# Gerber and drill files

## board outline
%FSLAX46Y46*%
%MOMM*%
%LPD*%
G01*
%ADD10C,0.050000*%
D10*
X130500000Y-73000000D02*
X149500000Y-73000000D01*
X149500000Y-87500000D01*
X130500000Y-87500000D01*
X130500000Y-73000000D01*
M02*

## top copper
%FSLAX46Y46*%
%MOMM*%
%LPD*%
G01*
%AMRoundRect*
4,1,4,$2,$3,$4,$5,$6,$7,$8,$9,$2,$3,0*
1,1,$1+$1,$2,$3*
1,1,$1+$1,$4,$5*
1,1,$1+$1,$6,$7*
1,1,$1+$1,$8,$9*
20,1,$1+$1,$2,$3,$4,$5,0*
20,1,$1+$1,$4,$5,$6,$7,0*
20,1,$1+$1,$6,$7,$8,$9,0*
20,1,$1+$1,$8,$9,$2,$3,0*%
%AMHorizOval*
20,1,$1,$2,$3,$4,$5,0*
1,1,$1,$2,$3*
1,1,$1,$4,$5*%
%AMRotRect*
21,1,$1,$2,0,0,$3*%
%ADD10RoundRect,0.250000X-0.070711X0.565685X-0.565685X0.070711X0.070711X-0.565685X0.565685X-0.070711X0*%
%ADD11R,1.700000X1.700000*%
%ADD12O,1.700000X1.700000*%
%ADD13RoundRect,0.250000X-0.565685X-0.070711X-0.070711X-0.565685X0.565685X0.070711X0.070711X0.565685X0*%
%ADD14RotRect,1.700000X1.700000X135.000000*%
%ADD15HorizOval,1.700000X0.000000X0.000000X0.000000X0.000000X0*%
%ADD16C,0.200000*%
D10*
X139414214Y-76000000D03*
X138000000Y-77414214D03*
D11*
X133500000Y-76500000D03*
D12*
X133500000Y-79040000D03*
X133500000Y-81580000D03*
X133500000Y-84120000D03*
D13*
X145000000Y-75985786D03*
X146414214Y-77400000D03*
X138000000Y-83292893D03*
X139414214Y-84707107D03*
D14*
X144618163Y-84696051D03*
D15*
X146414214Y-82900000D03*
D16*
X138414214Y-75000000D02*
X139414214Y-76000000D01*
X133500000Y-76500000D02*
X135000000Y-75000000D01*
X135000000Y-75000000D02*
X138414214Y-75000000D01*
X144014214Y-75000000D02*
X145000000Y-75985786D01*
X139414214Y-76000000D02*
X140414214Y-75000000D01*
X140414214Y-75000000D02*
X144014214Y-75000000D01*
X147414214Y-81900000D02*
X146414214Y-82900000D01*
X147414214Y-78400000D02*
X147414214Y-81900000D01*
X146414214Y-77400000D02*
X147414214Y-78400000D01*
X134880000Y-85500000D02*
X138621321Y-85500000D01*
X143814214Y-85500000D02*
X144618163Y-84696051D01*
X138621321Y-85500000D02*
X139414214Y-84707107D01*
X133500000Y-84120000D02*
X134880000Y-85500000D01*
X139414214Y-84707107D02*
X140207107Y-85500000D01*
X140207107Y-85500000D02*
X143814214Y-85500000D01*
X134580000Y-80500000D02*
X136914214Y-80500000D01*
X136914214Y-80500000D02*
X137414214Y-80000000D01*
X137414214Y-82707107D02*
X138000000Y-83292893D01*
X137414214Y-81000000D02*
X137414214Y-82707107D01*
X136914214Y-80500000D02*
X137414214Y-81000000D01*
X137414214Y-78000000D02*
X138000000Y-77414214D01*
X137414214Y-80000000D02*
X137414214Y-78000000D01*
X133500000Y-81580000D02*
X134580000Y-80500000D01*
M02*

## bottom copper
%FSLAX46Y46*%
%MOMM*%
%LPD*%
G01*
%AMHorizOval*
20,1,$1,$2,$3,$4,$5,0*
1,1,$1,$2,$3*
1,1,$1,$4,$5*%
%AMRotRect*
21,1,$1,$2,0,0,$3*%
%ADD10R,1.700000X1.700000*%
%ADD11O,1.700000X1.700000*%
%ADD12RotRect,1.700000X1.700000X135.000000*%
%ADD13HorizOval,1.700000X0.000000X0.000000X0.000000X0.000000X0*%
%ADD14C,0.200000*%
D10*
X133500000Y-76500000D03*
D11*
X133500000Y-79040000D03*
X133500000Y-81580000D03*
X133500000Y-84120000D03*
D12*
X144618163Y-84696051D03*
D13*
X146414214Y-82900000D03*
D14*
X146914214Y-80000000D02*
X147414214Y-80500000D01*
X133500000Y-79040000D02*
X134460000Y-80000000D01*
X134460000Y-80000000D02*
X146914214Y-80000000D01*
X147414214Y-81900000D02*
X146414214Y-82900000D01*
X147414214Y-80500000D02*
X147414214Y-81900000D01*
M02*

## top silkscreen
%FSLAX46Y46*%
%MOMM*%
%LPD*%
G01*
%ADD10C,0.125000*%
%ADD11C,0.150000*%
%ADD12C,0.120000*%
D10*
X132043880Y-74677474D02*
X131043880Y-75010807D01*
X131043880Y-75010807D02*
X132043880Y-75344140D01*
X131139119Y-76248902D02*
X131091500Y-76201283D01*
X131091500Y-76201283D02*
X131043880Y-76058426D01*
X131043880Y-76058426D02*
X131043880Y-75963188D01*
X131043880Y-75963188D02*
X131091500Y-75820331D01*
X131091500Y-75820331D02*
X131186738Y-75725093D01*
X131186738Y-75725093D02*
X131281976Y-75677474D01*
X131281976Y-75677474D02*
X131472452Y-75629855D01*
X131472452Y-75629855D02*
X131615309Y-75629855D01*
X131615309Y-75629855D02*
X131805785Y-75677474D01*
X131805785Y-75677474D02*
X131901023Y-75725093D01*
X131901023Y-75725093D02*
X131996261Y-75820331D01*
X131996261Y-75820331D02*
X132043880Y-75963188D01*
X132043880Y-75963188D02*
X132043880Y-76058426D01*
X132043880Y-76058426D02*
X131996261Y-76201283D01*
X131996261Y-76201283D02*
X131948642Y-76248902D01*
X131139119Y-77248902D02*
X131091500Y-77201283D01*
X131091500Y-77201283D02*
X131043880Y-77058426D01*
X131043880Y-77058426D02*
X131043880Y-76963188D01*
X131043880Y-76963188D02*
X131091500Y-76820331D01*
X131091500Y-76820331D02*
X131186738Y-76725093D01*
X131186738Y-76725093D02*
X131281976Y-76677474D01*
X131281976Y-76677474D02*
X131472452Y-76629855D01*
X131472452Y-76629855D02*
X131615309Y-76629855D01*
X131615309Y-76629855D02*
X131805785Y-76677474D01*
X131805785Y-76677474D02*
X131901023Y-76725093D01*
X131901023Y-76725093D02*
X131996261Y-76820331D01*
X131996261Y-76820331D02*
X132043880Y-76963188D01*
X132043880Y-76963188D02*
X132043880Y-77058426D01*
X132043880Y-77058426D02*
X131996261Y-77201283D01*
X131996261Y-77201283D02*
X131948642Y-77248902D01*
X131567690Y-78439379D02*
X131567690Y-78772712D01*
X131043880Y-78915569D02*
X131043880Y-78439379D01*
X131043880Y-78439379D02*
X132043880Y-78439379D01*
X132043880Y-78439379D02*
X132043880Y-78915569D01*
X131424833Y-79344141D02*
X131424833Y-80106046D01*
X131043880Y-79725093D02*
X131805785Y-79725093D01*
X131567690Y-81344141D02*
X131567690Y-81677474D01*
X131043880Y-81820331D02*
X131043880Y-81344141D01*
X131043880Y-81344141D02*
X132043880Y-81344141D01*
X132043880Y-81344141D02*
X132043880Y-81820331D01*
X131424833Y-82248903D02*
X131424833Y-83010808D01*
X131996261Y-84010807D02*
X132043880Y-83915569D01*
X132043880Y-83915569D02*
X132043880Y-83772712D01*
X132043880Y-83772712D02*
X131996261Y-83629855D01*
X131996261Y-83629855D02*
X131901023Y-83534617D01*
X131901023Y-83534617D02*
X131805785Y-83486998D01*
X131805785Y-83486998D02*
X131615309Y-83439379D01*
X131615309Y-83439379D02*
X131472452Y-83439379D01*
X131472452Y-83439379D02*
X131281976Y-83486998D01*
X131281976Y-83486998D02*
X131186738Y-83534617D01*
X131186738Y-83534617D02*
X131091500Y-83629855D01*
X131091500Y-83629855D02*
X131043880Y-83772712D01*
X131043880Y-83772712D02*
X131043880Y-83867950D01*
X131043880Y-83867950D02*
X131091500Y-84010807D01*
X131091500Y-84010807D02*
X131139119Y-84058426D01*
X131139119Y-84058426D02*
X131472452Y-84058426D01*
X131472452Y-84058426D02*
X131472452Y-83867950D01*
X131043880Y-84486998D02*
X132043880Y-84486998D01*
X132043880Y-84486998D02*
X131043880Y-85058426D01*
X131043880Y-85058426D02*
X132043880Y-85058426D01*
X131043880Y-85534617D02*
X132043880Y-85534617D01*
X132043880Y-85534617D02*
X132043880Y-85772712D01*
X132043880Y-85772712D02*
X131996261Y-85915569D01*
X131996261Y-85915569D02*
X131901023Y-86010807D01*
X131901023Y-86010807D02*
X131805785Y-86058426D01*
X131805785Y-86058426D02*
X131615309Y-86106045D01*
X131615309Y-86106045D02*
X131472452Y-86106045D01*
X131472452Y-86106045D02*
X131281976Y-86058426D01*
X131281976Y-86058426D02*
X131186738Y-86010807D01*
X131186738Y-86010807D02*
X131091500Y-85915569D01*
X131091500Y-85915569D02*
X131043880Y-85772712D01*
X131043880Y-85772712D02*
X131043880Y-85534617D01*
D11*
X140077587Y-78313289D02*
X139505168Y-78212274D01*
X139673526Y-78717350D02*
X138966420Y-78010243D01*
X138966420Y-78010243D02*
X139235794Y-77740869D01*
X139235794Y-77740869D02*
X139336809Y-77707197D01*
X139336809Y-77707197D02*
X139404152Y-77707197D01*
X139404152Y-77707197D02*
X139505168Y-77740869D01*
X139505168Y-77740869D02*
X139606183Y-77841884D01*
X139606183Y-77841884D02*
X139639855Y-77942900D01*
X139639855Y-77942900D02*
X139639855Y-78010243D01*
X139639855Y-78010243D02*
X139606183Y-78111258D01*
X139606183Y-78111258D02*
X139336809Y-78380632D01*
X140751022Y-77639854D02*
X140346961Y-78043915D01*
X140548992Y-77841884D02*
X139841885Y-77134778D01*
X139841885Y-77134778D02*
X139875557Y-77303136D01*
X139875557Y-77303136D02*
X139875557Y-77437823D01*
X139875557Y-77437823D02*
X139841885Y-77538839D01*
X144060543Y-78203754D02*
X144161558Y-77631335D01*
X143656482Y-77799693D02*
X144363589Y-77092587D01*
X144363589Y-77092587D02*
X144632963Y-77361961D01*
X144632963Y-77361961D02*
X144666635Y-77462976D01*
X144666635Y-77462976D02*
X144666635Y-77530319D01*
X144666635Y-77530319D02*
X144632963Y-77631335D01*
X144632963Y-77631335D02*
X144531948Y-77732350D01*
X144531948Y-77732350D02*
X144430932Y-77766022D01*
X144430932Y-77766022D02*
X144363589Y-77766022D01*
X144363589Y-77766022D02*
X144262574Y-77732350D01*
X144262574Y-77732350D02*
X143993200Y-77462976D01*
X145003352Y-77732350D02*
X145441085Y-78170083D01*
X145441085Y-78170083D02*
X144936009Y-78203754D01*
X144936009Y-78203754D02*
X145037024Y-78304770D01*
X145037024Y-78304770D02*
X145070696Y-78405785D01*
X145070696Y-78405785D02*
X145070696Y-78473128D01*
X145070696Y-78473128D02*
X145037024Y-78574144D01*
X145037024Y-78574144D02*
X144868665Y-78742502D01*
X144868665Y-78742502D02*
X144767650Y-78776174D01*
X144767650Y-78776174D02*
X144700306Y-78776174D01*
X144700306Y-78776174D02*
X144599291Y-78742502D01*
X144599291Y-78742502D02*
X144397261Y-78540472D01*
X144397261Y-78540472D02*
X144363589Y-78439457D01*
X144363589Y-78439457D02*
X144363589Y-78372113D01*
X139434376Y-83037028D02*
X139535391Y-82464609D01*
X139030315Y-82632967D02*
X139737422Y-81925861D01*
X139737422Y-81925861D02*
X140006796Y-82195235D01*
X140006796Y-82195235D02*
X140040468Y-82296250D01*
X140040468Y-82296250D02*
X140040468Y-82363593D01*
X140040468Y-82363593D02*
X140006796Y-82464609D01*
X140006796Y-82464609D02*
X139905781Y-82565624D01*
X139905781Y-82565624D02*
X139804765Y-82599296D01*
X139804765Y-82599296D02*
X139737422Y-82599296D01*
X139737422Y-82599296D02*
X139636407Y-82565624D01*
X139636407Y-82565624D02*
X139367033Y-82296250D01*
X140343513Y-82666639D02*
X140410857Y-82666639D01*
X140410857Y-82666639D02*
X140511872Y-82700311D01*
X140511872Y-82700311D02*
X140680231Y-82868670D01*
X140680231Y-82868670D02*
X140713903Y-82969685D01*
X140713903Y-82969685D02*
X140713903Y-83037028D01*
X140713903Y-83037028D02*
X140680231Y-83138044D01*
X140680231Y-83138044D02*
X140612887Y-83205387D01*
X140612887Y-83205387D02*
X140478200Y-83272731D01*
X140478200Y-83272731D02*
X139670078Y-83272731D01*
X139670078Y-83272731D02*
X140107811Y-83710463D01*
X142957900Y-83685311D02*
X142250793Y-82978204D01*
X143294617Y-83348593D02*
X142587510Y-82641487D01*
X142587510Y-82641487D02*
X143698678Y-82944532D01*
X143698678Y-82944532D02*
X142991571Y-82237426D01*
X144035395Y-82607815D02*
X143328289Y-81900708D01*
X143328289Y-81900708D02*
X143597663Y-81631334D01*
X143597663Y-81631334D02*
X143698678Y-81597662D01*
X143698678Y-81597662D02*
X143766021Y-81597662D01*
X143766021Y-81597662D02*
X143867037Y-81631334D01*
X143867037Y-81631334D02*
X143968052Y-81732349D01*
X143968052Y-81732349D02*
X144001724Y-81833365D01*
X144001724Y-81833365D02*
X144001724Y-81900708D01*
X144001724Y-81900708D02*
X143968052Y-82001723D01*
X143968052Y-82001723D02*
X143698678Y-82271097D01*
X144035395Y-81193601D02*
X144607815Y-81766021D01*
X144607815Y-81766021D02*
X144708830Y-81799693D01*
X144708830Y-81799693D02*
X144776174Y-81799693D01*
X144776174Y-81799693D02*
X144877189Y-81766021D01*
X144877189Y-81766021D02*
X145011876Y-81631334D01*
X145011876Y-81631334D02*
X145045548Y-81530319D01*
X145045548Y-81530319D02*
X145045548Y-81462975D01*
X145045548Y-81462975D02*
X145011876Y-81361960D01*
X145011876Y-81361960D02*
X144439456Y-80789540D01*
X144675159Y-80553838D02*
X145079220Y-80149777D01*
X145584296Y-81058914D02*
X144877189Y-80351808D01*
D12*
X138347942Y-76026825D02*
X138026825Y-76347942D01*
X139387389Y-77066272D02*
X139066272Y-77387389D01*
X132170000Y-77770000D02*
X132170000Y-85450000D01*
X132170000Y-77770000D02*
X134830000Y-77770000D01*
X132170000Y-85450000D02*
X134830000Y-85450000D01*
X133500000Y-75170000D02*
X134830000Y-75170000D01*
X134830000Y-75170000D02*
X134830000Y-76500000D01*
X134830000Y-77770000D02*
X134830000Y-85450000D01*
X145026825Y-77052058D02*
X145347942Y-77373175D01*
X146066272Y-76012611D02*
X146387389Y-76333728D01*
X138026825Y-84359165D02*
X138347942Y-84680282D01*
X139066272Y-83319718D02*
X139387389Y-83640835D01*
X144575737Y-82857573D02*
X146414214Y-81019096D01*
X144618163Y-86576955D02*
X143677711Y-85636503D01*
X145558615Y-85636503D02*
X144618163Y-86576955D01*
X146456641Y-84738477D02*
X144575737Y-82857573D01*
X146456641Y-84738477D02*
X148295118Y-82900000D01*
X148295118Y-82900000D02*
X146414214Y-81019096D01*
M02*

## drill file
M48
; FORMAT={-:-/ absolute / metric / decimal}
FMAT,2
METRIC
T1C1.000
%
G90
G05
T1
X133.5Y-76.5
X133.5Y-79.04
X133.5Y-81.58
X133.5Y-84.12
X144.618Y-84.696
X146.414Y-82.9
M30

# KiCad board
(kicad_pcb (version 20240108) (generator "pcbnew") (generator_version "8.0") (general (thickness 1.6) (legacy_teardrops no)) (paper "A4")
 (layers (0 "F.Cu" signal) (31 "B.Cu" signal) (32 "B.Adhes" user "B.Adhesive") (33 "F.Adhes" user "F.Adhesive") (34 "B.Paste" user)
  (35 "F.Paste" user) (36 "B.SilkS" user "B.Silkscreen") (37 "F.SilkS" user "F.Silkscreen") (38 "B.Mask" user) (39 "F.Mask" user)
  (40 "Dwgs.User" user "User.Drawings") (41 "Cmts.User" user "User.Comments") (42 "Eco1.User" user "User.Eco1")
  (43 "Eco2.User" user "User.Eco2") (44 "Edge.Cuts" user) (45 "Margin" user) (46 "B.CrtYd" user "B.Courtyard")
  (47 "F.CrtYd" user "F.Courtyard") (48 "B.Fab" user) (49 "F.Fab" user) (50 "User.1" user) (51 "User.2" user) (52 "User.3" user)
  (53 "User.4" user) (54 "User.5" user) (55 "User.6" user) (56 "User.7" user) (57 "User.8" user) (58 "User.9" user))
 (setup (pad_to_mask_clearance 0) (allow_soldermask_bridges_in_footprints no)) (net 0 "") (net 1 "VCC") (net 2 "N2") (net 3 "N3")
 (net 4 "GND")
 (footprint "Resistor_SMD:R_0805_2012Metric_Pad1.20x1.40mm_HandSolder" (layer "F.Cu") (at 138.707107 76.707107 -135)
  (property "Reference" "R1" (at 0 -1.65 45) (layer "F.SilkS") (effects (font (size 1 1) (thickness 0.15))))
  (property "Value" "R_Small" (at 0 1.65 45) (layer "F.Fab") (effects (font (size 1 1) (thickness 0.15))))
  (fp_line (start -0.227064 0.735) (end 0.227064 0.735) (stroke (width 0.12) (type solid)) (layer "F.SilkS"))
  (fp_line (start -0.227064 -0.735) (end 0.227064 -0.735) (stroke (width 0.12) (type solid)) (layer "F.SilkS"))
  (pad "1" smd roundrect (at -1 0 225) (size 1.2 1.4) (layers "F.Cu" "F.Paste" "F.Mask") (roundrect_rratio 0.208333) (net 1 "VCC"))
  (pad "2" smd roundrect (at 1 0 225) (size 1.2 1.4) (layers "F.Cu" "F.Paste" "F.Mask") (roundrect_rratio 0.208333) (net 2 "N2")))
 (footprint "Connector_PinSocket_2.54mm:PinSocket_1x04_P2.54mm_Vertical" (layer "F.Cu") (at 133.5 76.5)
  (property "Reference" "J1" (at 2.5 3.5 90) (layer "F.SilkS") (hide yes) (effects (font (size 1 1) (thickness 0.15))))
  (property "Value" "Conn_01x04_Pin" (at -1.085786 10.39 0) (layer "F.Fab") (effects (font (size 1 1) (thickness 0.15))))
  (fp_line (start -1.33 1.27) (end -1.33 8.95) (stroke (width 0.12) (type solid)) (layer "F.SilkS"))
  (fp_line (start -1.33 1.27) (end 1.33 1.27) (stroke (width 0.12) (type solid)) (layer "F.SilkS"))
  (fp_line (start -1.33 8.95) (end 1.33 8.95) (stroke (width 0.12) (type solid)) (layer "F.SilkS"))
  (fp_line (start 0 -1.33) (end 1.33 -1.33) (stroke (width 0.12) (type solid)) (layer "F.SilkS"))
  (fp_line (start 1.33 -1.33) (end 1.33 0) (stroke (width 0.12) (type solid)) (layer "F.SilkS"))
  (fp_line (start 1.33 1.27) (end 1.33 8.95) (stroke (width 0.12) (type solid)) (layer "F.SilkS"))
  (pad "1" thru_hole rect (at 0 0) (size 1.7 1.7) (drill 1) (layers "*.Cu" "*.Mask") (remove_unused_layers no) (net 1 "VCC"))
  (pad "2" thru_hole oval (at 0 2.54) (size 1.7 1.7) (drill 1) (layers "*.Cu" "*.Mask") (remove_unused_layers no) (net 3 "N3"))
  (pad "3" thru_hole oval (at 0 5.08) (size 1.7 1.7) (drill 1) (layers "*.Cu" "*.Mask") (remove_unused_layers no) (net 2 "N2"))
  (pad "4" thru_hole oval (at 0 7.62) (size 1.7 1.7) (drill 1) (layers "*.Cu" "*.Mask") (remove_unused_layers no) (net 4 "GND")))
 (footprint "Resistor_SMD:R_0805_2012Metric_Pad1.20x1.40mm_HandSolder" (layer "F.Cu") (at 145.707107 76.692893 -45)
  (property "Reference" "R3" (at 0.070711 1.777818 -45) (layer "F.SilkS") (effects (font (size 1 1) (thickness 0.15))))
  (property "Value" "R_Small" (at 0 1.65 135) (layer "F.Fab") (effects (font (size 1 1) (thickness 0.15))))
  (fp_line (start -0.227064 0.735) (end 0.227064 0.735) (stroke (width 0.12) (type solid)) (layer "F.SilkS"))
  (fp_line (start -0.227064 -0.735) (end 0.227064 -0.735) (stroke (width 0.12) (type solid)) (layer "F.SilkS"))
  (pad "1" smd roundrect (at -1 0 315) (size 1.2 1.4) (layers "F.Cu" "F.Paste" "F.Mask") (roundrect_rratio 0.208333) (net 1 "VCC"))
  (pad "2" smd roundrect (at 1 0 315) (size 1.2 1.4) (layers "F.Cu" "F.Paste" "F.Mask") (roundrect_rratio 0.208333) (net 3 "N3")))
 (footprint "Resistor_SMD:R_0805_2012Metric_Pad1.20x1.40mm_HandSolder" (layer "F.Cu") (at 138.707107 84 -45)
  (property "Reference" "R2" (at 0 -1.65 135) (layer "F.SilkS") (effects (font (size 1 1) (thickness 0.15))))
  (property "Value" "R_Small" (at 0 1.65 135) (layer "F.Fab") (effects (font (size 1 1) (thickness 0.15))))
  (fp_line (start -0.227064 0.735) (end 0.227064 0.735) (stroke (width 0.12) (type solid)) (layer "F.SilkS"))
  (fp_line (start -0.227064 -0.735) (end 0.227064 -0.735) (stroke (width 0.12) (type solid)) (layer "F.SilkS"))
  (pad "1" smd roundrect (at -1 0 315) (size 1.2 1.4) (layers "F.Cu" "F.Paste" "F.Mask") (roundrect_rratio 0.208333) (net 2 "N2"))
  (pad "2" smd roundrect (at 1 0 315) (size 1.2 1.4) (layers "F.Cu" "F.Paste" "F.Mask") (roundrect_rratio 0.208333) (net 4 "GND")))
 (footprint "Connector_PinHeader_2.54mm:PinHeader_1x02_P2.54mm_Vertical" (layer "F.Cu") (at 144.618163 84.696051 135)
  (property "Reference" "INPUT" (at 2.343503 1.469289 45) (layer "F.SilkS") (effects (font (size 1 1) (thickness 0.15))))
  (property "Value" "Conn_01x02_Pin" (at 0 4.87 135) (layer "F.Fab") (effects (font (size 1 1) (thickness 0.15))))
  (fp_line (start 1.33 1.270001) (end 1.33 3.87) (stroke (width 0.12) (type solid)) (layer "F.SilkS"))
  (fp_line (start -1.33 -1.33) (end 0 -1.33) (stroke (width 0.12) (type solid)) (layer "F.SilkS"))
  (fp_line (start -1.33 0) (end -1.33 -1.33) (stroke (width 0.12) (type solid)) (layer "F.SilkS"))
  (fp_line (start -1.33 1.270001) (end 1.33 1.270001) (stroke (width 0.12) (type solid)) (layer "F.SilkS"))
  (fp_line (start -1.33 1.270001) (end -1.33 3.87) (stroke (width 0.12) (type solid)) (layer "F.SilkS"))
  (fp_line (start -1.33 3.87) (end 1.33 3.87) (stroke (width 0.12) (type solid)) (layer "F.SilkS"))
  (pad "1" thru_hole rect (at 0 0 135) (size 1.7 1.7) (drill 1) (layers "*.Cu" "*.Mask") (remove_unused_layers no) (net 4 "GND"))
  (pad "2" thru_hole oval (at 0 2.54 135) (size 1.7 1.7) (drill 1) (layers "*.Cu" "*.Mask") (remove_unused_layers no) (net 3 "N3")))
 (gr_rect (start 130.5 73) (end 149.5 87.5) (stroke (width 0.05) (type default)) (fill none) (layer "Edge.Cuts"))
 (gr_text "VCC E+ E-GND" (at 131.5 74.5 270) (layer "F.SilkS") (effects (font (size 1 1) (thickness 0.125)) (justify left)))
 (segment (start 138.414214 75) (end 139.414214 76) (width 0.2) (layer "F.Cu") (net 1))
 (segment (start 133.5 76.5) (end 135 75) (width 0.2) (layer "F.Cu") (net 1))
 (segment (start 135 75) (end 138.414214 75) (width 0.2) (layer "F.Cu") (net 1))
 (segment (start 144.014214 75) (end 145 75.985786) (width 0.2) (layer "F.Cu") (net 1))
 (segment (start 139.414214 76) (end 140.414214 75) (width 0.2) (layer "F.Cu") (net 1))
 (segment (start 140.414214 75) (end 144.014214 75) (width 0.2) (layer "F.Cu") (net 1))
 (segment (start 147.414214 81.9) (end 146.414214 82.9) (width 0.2) (layer "F.Cu") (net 3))
 (segment (start 147.414214 78.4) (end 147.414214 81.9) (width 0.2) (layer "F.Cu") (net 3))
 (segment (start 146.414214 77.4) (end 147.414214 78.4) (width 0.2) (layer "F.Cu") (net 3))
 (segment (start 146.914214 80) (end 147.414214 80.5) (width 0.2) (layer "B.Cu") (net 3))
 (segment (start 133.5 79.04) (end 134.46 80) (width 0.2) (layer "B.Cu") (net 3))
 (segment (start 134.46 80) (end 146.914214 80) (width 0.2) (layer "B.Cu") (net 3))
 (segment (start 147.414214 81.9) (end 146.414214 82.9) (width 0.2) (layer "B.Cu") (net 3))
 (segment (start 147.414214 80.5) (end 147.414214 81.9) (width 0.2) (layer "B.Cu") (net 3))
 (segment (start 134.88 85.5) (end 138.621321 85.5) (width 0.2) (layer "F.Cu") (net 4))
 (segment (start 143.814214 85.5) (end 144.618163 84.696051) (width 0.2) (layer "F.Cu") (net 4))
 (segment (start 138.621321 85.5) (end 139.414214 84.707107) (width 0.2) (layer "F.Cu") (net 4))
 (segment (start 133.5 84.12) (end 134.88 85.5) (width 0.2) (layer "F.Cu") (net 4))
 (segment (start 139.414214 84.707107) (end 140.207107 85.5) (width 0.2) (layer "F.Cu") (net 4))
 (segment (start 140.207107 85.5) (end 143.814214 85.5) (width 0.2) (layer "F.Cu") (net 4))
 (segment (start 134.58 80.5) (end 136.914214 80.5) (width 0.2) (layer "F.Cu") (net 2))
 (segment (start 136.914214 80.5) (end 137.414214 80) (width 0.2) (layer "F.Cu") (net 2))
 (segment (start 137.414214 82.707107) (end 138 83.292893) (width 0.2) (layer "F.Cu") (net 2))
 (segment (start 137.414214 81) (end 137.414214 82.707107) (width 0.2) (layer "F.Cu") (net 2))
 (segment (start 136.914214 80.5) (end 137.414214 81) (width 0.2) (layer "F.Cu") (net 2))
 (segment (start 137.414214 78) (end 138 77.414214) (width 0.2) (layer "F.Cu") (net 2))
 (segment (start 137.414214 80) (end 137.414214 78) (width 0.2) (layer "F.Cu") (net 2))
 (segment (start 133.5 81.58) (end 134.58 80.5) (width 0.2) (layer "F.Cu") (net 2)))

